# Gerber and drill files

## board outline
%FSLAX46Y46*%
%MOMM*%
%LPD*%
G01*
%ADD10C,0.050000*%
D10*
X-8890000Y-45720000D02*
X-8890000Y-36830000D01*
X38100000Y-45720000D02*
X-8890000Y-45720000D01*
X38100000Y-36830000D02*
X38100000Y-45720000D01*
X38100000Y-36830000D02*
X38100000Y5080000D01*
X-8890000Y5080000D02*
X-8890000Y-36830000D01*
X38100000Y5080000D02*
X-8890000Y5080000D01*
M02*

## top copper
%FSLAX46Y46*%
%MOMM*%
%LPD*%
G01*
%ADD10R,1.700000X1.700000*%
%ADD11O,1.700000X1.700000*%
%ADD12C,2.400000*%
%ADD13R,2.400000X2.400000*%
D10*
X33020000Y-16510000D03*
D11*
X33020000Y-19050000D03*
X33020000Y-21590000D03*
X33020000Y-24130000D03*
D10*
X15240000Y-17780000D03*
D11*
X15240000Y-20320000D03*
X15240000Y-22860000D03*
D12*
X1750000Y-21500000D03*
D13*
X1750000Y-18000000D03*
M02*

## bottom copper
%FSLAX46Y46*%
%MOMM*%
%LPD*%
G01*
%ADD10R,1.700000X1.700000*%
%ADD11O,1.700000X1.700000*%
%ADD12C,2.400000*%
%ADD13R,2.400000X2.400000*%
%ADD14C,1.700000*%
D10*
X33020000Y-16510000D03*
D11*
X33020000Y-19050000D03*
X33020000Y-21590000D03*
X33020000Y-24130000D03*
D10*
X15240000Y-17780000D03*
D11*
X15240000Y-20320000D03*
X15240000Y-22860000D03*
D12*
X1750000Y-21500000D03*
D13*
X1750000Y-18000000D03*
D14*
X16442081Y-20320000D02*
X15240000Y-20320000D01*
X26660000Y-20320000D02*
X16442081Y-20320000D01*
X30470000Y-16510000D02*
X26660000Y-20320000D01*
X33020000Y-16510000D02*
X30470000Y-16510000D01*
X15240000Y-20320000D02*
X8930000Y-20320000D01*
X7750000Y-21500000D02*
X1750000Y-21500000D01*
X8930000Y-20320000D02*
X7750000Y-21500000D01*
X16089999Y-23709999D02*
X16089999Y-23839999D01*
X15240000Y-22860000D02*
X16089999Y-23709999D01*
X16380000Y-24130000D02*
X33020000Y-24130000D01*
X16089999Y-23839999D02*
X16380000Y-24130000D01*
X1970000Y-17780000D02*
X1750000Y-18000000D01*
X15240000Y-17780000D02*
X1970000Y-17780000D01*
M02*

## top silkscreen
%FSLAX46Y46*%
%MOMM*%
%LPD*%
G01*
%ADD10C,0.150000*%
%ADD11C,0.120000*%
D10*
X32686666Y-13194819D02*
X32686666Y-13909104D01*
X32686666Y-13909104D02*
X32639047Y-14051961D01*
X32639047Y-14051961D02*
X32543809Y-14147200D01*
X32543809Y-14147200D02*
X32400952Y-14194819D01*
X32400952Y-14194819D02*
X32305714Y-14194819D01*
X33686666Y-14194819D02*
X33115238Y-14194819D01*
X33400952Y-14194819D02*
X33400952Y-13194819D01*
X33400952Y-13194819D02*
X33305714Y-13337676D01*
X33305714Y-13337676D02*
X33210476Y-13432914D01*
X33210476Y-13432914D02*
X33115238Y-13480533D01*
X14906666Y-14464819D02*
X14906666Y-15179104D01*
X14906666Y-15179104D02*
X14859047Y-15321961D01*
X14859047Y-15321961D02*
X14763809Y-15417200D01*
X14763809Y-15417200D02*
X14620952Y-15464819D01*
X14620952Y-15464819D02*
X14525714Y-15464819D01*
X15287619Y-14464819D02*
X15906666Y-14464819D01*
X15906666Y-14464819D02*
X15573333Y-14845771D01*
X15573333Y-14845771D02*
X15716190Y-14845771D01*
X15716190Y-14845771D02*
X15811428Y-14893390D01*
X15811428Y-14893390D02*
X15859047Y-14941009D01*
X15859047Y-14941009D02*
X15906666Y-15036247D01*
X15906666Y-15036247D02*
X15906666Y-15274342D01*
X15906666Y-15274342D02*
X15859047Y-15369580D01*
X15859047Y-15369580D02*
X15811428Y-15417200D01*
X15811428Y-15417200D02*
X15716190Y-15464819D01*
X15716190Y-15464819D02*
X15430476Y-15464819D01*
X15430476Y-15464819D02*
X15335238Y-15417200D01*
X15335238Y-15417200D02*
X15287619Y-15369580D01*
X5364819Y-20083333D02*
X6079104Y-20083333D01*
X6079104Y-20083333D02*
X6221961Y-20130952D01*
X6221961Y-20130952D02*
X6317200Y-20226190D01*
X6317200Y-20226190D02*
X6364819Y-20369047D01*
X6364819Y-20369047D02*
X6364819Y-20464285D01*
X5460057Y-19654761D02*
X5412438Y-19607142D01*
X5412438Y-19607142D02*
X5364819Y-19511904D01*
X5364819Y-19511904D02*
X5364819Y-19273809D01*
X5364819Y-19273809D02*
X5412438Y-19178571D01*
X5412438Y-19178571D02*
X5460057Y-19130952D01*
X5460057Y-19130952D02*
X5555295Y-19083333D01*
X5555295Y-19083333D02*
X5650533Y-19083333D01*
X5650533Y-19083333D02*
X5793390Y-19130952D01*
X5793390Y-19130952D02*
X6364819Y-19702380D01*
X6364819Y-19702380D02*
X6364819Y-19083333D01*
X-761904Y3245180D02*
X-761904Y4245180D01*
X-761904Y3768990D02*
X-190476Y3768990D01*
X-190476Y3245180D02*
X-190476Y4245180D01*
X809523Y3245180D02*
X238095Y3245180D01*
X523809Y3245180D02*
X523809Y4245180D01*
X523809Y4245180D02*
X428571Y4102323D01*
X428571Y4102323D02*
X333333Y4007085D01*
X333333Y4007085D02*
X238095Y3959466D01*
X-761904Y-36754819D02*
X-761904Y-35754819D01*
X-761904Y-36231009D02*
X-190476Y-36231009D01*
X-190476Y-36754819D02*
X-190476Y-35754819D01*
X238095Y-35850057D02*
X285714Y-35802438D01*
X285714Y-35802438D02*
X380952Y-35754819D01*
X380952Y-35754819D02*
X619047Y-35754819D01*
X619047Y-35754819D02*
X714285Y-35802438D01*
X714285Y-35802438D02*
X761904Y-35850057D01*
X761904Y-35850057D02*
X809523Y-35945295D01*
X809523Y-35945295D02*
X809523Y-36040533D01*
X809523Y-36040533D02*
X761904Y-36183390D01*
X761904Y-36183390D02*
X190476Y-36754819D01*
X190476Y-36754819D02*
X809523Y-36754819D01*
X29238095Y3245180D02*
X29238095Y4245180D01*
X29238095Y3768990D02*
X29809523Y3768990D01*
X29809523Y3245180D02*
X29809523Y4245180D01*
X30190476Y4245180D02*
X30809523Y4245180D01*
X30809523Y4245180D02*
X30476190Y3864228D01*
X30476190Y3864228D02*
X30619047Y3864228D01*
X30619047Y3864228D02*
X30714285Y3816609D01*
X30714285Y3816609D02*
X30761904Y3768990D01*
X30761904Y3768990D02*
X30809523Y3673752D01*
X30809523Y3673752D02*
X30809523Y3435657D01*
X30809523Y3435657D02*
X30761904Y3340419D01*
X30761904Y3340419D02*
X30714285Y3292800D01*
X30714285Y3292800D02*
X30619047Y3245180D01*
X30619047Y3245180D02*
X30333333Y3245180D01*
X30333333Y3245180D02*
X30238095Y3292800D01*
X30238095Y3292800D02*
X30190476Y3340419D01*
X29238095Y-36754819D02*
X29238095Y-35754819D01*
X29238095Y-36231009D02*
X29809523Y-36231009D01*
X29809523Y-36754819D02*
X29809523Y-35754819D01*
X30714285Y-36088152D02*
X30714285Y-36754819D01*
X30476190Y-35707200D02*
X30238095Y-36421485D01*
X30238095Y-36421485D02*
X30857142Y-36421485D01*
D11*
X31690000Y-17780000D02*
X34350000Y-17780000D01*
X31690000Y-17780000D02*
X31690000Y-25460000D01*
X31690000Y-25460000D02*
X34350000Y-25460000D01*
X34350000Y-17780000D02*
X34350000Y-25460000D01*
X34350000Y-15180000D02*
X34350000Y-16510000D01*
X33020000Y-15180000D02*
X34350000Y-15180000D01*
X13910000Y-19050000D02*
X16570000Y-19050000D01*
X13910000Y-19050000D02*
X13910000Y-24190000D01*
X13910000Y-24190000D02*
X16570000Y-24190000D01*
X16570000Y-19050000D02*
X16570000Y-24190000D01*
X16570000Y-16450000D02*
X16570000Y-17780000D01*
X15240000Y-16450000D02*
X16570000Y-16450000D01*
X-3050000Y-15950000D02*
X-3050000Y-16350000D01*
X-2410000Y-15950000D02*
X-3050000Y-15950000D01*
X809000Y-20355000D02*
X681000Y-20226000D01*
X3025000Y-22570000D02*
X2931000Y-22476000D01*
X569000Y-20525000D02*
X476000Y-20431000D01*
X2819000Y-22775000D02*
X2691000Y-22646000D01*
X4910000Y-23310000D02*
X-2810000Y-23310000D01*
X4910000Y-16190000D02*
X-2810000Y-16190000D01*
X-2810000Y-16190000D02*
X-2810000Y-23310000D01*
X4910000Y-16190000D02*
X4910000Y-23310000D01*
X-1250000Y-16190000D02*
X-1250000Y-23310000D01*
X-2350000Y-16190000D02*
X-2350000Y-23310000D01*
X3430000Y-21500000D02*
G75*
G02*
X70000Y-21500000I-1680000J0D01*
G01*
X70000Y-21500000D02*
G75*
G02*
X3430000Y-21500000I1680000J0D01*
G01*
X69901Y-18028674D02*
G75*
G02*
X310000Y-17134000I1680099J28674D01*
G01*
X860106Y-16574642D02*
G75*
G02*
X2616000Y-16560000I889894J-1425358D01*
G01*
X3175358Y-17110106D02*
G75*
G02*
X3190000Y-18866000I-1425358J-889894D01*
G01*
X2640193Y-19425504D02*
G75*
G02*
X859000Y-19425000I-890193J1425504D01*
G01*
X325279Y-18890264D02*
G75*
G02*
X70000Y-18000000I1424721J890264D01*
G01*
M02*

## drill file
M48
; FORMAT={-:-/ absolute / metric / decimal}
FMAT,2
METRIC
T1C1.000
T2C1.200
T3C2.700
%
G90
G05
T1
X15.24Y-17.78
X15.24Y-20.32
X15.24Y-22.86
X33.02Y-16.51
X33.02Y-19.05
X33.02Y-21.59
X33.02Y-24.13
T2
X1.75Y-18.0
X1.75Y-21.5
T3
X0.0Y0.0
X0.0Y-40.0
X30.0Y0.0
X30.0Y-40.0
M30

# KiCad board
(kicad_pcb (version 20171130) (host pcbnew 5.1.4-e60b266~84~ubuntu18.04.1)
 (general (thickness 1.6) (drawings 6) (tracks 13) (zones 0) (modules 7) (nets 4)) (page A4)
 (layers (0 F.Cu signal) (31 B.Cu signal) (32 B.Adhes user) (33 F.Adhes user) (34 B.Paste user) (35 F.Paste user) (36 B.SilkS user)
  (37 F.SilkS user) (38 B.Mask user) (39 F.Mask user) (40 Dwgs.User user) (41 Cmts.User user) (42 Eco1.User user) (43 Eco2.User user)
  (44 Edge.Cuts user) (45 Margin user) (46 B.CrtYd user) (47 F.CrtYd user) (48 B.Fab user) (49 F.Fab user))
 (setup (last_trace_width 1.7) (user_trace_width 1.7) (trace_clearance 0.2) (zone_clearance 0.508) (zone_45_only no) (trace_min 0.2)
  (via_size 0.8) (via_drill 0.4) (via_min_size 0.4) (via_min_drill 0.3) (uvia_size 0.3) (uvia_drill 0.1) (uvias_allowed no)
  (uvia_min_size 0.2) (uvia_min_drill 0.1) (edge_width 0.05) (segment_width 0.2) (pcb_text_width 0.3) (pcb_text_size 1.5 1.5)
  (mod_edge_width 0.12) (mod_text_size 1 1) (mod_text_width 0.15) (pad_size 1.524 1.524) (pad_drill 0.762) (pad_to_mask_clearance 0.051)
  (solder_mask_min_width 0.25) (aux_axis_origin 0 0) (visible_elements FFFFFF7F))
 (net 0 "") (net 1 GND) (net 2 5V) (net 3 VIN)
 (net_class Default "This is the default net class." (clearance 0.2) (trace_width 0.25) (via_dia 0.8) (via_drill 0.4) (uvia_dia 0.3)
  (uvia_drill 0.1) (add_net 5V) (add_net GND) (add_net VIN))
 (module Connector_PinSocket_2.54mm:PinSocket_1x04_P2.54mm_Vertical (layer F.Cu) (at 33.02 16.51)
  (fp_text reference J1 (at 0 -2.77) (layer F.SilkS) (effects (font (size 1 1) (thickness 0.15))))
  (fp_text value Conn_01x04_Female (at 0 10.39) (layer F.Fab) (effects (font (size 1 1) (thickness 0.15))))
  (fp_line (start -1.33 1.27) (end 1.33 1.27) (layer F.SilkS) (width 0.12))
  (fp_line (start -1.33 1.27) (end -1.33 8.95) (layer F.SilkS) (width 0.12))
  (fp_line (start -1.33 8.95) (end 1.33 8.95) (layer F.SilkS) (width 0.12))
  (fp_line (start 1.33 1.27) (end 1.33 8.95) (layer F.SilkS) (width 0.12))
  (fp_line (start 1.33 -1.33) (end 1.33 0) (layer F.SilkS) (width 0.12))
  (fp_line (start 0 -1.33) (end 1.33 -1.33) (layer F.SilkS) (width 0.12))
  (pad 1 thru_hole rect (at 0 0) (size 1.7 1.7) (drill 1) (layers *.Cu *.Mask) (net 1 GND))
  (pad 2 thru_hole oval (at 0 2.54) (size 1.7 1.7) (drill 1) (layers *.Cu *.Mask))
  (pad 3 thru_hole oval (at 0 5.08) (size 1.7 1.7) (drill 1) (layers *.Cu *.Mask))
  (pad 4 thru_hole oval (at 0 7.62) (size 1.7 1.7) (drill 1) (layers *.Cu *.Mask) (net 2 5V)))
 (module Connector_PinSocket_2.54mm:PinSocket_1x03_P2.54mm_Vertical (layer F.Cu) (at 15.24 17.78)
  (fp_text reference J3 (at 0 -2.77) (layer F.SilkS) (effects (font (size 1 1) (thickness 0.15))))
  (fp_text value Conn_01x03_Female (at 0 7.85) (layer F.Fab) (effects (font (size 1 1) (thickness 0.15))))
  (fp_line (start -1.33 1.27) (end 1.33 1.27) (layer F.SilkS) (width 0.12))
  (fp_line (start -1.33 1.27) (end -1.33 6.41) (layer F.SilkS) (width 0.12))
  (fp_line (start -1.33 6.41) (end 1.33 6.41) (layer F.SilkS) (width 0.12))
  (fp_line (start 1.33 1.27) (end 1.33 6.41) (layer F.SilkS) (width 0.12))
  (fp_line (start 1.33 -1.33) (end 1.33 0) (layer F.SilkS) (width 0.12))
  (fp_line (start 0 -1.33) (end 1.33 -1.33) (layer F.SilkS) (width 0.12))
  (pad 1 thru_hole rect (at 0 0) (size 1.7 1.7) (drill 1) (layers *.Cu *.Mask) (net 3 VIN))
  (pad 2 thru_hole oval (at 0 2.54) (size 1.7 1.7) (drill 1) (layers *.Cu *.Mask) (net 1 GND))
  (pad 3 thru_hole oval (at 0 5.08) (size 1.7 1.7) (drill 1) (layers *.Cu *.Mask) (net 2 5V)))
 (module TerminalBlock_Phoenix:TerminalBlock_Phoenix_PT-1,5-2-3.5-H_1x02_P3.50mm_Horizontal (layer F.Cu) (at 1.75 18 270)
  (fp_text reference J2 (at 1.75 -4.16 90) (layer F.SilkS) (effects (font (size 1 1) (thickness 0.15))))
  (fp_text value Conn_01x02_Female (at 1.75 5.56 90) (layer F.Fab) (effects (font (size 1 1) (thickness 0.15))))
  (fp_line (start -2.05 4.8) (end -1.65 4.8) (layer F.SilkS) (width 0.12))
  (fp_line (start -2.05 4.16) (end -2.05 4.8) (layer F.SilkS) (width 0.12))
  (fp_line (start 2.355 0.941) (end 2.226 1.069) (layer F.SilkS) (width 0.12))
  (fp_line (start 4.57 -1.275) (end 4.476 -1.181) (layer F.SilkS) (width 0.12))
  (fp_line (start 2.525 1.181) (end 2.431 1.274) (layer F.SilkS) (width 0.12))
  (fp_line (start 4.775 -1.069) (end 4.646 -0.941) (layer F.SilkS) (width 0.12))
  (fp_line (start 5.31 -3.16) (end 5.31 4.56) (layer F.SilkS) (width 0.12))
  (fp_line (start -1.81 -3.16) (end -1.81 4.56) (layer F.SilkS) (width 0.12))
  (fp_line (start -1.81 4.56) (end 5.31 4.56) (layer F.SilkS) (width 0.12))
  (fp_line (start -1.81 -3.16) (end 5.31 -3.16) (layer F.SilkS) (width 0.12))
  (fp_line (start -1.81 3) (end 5.31 3) (layer F.SilkS) (width 0.12))
  (fp_line (start -1.81 4.1) (end 5.31 4.1) (layer F.SilkS) (width 0.12))
  (fp_circle (center 3.5 0) (end 5.18 0) (layer F.SilkS) (width 0.12))
  (fp_arc (start 0 0) (end -0.866 1.44) (angle -32) (layer F.SilkS) (width 0.12))
  (fp_arc (start 0 0) (end -1.44 -0.866) (angle -63) (layer F.SilkS) (width 0.12))
  (fp_arc (start 0 0) (end 0.866 -1.44) (angle -63) (layer F.SilkS) (width 0.12))
  (fp_arc (start 0 0) (end 1.425 0.891) (angle -64) (layer F.SilkS) (width 0.12))
  (fp_arc (start 0 0) (end 0 1.68) (angle -32) (layer F.SilkS) (width 0.12))
  (pad 2 thru_hole circle (at 3.5 0 270) (size 2.4 2.4) (drill 1.2) (layers *.Cu *.Mask) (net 1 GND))
  (pad 1 thru_hole rect (at 0 0 270) (size 2.4 2.4) (drill 1.2) (layers *.Cu *.Mask) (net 3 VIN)))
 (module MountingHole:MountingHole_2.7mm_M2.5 (layer F.Cu) (at 0 0)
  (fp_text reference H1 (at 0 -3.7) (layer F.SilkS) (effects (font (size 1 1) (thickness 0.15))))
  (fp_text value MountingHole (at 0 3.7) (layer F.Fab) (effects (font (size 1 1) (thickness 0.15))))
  (pad 1 np_thru_hole circle (at 0 0) (size 2.7 2.7) (drill 2.7) (layers *.Cu *.Mask)))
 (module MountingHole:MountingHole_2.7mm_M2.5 (layer F.Cu) (at 0 40)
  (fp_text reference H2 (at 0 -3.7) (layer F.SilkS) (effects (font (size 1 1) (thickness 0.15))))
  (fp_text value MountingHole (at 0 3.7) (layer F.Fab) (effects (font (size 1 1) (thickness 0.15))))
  (pad 1 np_thru_hole circle (at 0 0) (size 2.7 2.7) (drill 2.7) (layers *.Cu *.Mask)))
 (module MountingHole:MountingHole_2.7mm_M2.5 (layer F.Cu) (at 30 0)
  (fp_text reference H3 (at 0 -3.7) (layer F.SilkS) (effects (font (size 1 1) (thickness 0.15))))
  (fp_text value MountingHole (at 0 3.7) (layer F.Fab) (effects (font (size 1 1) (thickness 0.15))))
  (pad 1 np_thru_hole circle (at 0 0) (size 2.7 2.7) (drill 2.7) (layers *.Cu *.Mask)))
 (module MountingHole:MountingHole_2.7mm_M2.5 (layer F.Cu) (at 30 40)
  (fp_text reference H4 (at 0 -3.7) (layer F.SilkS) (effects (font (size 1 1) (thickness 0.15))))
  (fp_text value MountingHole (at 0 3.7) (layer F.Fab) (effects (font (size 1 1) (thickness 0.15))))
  (pad 1 np_thru_hole circle (at 0 0) (size 2.7 2.7) (drill 2.7) (layers *.Cu *.Mask)))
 (gr_line (start -8.89 45.72) (end -8.89 36.83) (layer Edge.Cuts) (width 0.05))
 (gr_line (start 38.1 45.72) (end -8.89 45.72) (layer Edge.Cuts) (width 0.05))
 (gr_line (start 38.1 36.83) (end 38.1 45.72) (layer Edge.Cuts) (width 0.05))
 (gr_line (start 38.1 36.83) (end 38.1 -5.08) (layer Edge.Cuts) (width 0.05))
 (gr_line (start -8.89 -5.08) (end -8.89 36.83) (layer Edge.Cuts) (width 0.05))
 (gr_line (start 38.1 -5.08) (end -8.89 -5.08) (layer Edge.Cuts) (width 0.05))
 (segment (start 16.442081 20.32) (end 15.24 20.32) (width 1.7) (layer B.Cu) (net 1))
 (segment (start 26.66 20.32) (end 16.442081 20.32) (width 1.7) (layer B.Cu) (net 1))
 (segment (start 30.47 16.51) (end 26.66 20.32) (width 1.7) (layer B.Cu) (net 1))
 (segment (start 33.02 16.51) (end 30.47 16.51) (width 1.7) (layer B.Cu) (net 1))
 (segment (start 15.24 20.32) (end 8.93 20.32) (width 1.7) (layer B.Cu) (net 1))
 (segment (start 7.75 21.5) (end 1.75 21.5) (width 1.7) (layer B.Cu) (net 1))
 (segment (start 8.93 20.32) (end 7.75 21.5) (width 1.7) (layer B.Cu) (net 1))
 (segment (start 16.089999 23.709999) (end 16.089999 23.839999) (width 1.7) (layer B.Cu) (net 2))
 (segment (start 15.24 22.86) (end 16.089999 23.709999) (width 1.7) (layer B.Cu) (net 2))
 (segment (start 16.38 24.13) (end 33.02 24.13) (width 1.7) (layer B.Cu) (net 2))
 (segment (start 16.089999 23.839999) (end 16.38 24.13) (width 1.7) (layer B.Cu) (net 2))
 (segment (start 1.97 17.78) (end 1.75 18) (width 1.7) (layer B.Cu) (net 3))
 (segment (start 15.24 17.78) (end 1.97 17.78) (width 1.7) (layer B.Cu) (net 3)))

